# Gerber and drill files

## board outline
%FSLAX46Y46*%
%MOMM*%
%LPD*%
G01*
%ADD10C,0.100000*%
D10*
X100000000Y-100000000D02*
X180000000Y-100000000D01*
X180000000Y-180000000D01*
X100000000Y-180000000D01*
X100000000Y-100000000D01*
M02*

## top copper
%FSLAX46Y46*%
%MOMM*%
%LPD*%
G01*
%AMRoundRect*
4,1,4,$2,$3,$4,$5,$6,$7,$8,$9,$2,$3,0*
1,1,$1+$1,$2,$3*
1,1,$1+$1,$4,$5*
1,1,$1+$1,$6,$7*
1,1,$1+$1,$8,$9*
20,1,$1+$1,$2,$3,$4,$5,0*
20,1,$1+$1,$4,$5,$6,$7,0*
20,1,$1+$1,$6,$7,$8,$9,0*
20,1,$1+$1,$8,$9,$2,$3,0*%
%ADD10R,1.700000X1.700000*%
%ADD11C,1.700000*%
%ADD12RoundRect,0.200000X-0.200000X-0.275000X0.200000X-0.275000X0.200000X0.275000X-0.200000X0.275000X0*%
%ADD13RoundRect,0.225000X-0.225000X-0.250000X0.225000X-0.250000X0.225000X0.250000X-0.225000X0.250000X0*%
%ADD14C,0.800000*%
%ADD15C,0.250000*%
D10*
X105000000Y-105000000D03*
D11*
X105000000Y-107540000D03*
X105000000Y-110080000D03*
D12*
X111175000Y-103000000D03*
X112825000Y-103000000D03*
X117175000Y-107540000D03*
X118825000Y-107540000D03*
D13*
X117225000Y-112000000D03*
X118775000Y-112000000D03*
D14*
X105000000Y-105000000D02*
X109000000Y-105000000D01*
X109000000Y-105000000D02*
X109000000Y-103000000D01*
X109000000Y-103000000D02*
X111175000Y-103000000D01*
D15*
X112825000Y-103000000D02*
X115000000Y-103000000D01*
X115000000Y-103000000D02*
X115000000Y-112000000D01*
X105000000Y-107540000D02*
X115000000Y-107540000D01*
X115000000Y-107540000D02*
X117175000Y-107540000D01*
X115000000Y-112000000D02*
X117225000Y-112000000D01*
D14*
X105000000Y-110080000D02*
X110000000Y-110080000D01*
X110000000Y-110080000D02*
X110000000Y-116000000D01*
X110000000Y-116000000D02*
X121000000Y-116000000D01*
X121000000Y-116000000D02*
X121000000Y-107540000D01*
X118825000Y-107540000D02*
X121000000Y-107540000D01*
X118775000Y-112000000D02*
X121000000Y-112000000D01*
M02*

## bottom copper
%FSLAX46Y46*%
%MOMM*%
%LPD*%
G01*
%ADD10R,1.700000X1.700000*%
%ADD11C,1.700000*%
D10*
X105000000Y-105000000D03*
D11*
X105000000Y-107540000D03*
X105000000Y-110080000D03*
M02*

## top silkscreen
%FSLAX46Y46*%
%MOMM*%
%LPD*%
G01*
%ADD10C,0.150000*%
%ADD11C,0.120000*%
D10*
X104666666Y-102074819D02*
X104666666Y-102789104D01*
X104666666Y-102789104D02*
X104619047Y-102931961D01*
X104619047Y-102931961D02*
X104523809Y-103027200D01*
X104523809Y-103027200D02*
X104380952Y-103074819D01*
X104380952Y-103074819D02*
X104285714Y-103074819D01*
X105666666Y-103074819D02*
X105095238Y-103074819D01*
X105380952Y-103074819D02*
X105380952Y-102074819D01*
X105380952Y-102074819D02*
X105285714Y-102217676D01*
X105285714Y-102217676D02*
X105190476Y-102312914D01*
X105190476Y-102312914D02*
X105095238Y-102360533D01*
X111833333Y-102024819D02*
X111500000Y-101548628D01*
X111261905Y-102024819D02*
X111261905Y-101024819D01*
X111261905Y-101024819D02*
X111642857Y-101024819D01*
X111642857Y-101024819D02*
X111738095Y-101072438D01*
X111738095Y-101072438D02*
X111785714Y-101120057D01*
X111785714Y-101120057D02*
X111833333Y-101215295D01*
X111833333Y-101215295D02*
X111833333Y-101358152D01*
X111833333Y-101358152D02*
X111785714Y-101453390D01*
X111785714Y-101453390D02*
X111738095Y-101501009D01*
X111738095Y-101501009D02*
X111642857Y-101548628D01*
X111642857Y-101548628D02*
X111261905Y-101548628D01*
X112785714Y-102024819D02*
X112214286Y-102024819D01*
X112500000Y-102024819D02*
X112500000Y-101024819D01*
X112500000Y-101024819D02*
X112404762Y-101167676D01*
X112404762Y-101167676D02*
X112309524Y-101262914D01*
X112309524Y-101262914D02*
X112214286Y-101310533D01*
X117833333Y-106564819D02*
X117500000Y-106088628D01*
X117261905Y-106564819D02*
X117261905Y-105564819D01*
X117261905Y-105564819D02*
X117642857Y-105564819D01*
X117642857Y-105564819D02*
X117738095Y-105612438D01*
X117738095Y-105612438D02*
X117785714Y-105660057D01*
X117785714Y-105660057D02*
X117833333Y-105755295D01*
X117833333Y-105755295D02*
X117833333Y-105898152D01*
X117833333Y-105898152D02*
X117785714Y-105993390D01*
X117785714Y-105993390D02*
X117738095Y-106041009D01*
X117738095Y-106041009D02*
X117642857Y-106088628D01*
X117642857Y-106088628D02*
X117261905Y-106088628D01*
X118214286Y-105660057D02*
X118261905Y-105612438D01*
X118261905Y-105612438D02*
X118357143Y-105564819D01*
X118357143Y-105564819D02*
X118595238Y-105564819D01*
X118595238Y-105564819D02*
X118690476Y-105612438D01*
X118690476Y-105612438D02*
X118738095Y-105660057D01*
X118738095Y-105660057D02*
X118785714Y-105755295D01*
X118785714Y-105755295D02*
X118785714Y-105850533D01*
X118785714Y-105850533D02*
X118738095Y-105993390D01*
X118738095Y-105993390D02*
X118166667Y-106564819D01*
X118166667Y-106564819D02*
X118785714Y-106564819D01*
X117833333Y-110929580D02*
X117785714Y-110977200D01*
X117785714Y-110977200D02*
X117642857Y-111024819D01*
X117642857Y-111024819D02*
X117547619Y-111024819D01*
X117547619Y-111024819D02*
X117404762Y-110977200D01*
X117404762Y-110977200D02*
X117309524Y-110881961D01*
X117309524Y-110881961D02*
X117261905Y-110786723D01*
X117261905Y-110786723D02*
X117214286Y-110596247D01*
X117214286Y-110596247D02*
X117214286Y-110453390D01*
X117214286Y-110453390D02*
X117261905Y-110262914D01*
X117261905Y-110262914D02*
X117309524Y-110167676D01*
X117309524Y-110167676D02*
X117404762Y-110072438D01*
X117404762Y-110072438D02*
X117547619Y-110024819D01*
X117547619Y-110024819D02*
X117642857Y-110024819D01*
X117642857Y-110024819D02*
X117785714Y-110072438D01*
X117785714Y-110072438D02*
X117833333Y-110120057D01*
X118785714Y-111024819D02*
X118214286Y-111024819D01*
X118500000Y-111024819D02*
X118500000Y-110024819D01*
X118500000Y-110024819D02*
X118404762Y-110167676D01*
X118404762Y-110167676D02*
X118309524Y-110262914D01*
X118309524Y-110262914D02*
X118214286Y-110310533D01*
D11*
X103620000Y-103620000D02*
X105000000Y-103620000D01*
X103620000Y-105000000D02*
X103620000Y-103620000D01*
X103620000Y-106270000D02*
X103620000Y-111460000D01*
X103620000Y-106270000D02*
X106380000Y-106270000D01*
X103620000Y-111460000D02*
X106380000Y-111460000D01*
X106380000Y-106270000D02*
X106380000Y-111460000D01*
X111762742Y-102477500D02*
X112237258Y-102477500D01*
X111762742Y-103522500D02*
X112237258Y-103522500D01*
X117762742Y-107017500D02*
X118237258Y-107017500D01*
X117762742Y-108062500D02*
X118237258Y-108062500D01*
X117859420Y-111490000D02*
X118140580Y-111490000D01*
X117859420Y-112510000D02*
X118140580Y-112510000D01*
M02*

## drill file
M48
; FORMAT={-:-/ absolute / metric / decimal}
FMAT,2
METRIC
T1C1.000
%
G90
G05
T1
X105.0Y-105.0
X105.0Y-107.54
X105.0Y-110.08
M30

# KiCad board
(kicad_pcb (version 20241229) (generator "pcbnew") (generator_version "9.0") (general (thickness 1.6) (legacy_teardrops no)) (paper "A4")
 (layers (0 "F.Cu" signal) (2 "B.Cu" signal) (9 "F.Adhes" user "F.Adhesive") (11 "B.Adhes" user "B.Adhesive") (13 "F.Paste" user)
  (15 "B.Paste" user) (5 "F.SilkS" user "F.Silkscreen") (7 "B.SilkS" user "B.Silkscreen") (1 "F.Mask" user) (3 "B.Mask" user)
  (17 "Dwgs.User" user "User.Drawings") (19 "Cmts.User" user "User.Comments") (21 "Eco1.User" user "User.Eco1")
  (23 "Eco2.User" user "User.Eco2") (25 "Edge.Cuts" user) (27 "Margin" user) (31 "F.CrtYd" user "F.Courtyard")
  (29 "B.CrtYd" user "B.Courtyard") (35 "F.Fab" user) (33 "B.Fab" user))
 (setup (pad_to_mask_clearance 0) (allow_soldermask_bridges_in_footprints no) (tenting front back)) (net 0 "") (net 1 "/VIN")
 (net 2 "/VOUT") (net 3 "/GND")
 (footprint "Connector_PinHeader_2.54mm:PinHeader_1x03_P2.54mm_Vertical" (layer "F.Cu") (at 105 105)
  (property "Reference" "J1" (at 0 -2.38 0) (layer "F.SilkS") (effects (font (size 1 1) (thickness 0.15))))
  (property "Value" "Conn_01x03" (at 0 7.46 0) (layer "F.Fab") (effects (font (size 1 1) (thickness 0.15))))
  (fp_line (start -1.38 -1.38) (end 0 -1.38) (stroke (width 0.12) (type solid)) (layer "F.SilkS"))
  (fp_line (start -1.38 0) (end -1.38 -1.38) (stroke (width 0.12) (type solid)) (layer "F.SilkS"))
  (fp_line (start -1.38 1.27) (end -1.38 6.46) (stroke (width 0.12) (type solid)) (layer "F.SilkS"))
  (fp_line (start -1.38 1.27) (end 1.38 1.27) (stroke (width 0.12) (type solid)) (layer "F.SilkS"))
  (fp_line (start -1.38 6.46) (end 1.38 6.46) (stroke (width 0.12) (type solid)) (layer "F.SilkS"))
  (fp_line (start 1.38 1.27) (end 1.38 6.46) (stroke (width 0.12) (type solid)) (layer "F.SilkS"))
  (pad "1" thru_hole rect (at 0 0) (size 1.7 1.7) (drill 1) (layers "*.Cu" "*.Mask") (remove_unused_layers no) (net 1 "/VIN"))
  (pad "2" thru_hole circle (at 0 2.54) (size 1.7 1.7) (drill 1) (layers "*.Cu" "*.Mask") (remove_unused_layers no) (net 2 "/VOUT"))
  (pad "3" thru_hole circle (at 0 5.08) (size 1.7 1.7) (drill 1) (layers "*.Cu" "*.Mask") (remove_unused_layers no) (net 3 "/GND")))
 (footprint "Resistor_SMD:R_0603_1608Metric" (layer "F.Cu") (at 112 103)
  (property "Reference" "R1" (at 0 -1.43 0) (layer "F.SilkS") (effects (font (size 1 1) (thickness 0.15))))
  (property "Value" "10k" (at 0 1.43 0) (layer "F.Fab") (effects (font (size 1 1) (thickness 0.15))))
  (fp_line (start -0.237258 -0.5225) (end 0.237258 -0.5225) (stroke (width 0.12) (type solid)) (layer "F.SilkS"))
  (fp_line (start -0.237258 0.5225) (end 0.237258 0.5225) (stroke (width 0.12) (type solid)) (layer "F.SilkS"))
  (pad "1" smd roundrect (at -0.825 0) (size 0.8 0.95) (layers "F.Cu" "F.Mask" "F.Paste") (roundrect_rratio 0.25) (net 1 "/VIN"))
  (pad "2" smd roundrect (at 0.825 0) (size 0.8 0.95) (layers "F.Cu" "F.Mask" "F.Paste") (roundrect_rratio 0.25) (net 2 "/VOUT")))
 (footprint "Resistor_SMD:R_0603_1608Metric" (layer "F.Cu") (at 118 107.54)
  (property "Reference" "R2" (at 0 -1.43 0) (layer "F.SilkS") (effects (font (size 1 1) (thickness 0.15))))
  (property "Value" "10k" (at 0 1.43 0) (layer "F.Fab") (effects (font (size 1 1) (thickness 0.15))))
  (fp_line (start -0.237258 -0.5225) (end 0.237258 -0.5225) (stroke (width 0.12) (type solid)) (layer "F.SilkS"))
  (fp_line (start -0.237258 0.5225) (end 0.237258 0.5225) (stroke (width 0.12) (type solid)) (layer "F.SilkS"))
  (pad "1" smd roundrect (at -0.825 0) (size 0.8 0.95) (layers "F.Cu" "F.Mask" "F.Paste") (roundrect_rratio 0.25) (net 2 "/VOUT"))
  (pad "2" smd roundrect (at 0.825 0) (size 0.8 0.95) (layers "F.Cu" "F.Mask" "F.Paste") (roundrect_rratio 0.25) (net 3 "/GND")))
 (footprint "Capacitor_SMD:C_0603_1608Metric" (layer "F.Cu") (at 118 112)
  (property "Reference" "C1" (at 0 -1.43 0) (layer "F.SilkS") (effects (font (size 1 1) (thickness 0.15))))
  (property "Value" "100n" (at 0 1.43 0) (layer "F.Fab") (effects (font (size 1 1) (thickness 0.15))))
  (fp_line (start -0.14058 -0.51) (end 0.14058 -0.51) (stroke (width 0.12) (type solid)) (layer "F.SilkS"))
  (fp_line (start -0.14058 0.51) (end 0.14058 0.51) (stroke (width 0.12) (type solid)) (layer "F.SilkS"))
  (pad "1" smd roundrect (at -0.775 0) (size 0.9 0.95) (layers "F.Cu" "F.Mask" "F.Paste") (roundrect_rratio 0.25) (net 2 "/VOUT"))
  (pad "2" smd roundrect (at 0.775 0) (size 0.9 0.95) (layers "F.Cu" "F.Mask" "F.Paste") (roundrect_rratio 0.25) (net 3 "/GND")))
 (gr_rect (start 100 100) (end 180 180) (stroke (width 0.1) (type default)) (fill no) (layer "Edge.Cuts"))
 (segment (start 105 105) (end 109 105) (width 0.8) (layer "F.Cu") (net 1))
 (segment (start 109 105) (end 109 103) (width 0.8) (layer "F.Cu") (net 1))
 (segment (start 109 103) (end 111.175 103) (width 0.8) (layer "F.Cu") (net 1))
 (segment (start 112.825 103) (end 115 103) (width 0.25) (layer "F.Cu") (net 2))
 (segment (start 115 103) (end 115 112) (width 0.25) (layer "F.Cu") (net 2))
 (segment (start 105 107.54) (end 115 107.54) (width 0.25) (layer "F.Cu") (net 2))
 (segment (start 115 107.54) (end 117.175 107.54) (width 0.25) (layer "F.Cu") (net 2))
 (segment (start 115 112) (end 117.225 112) (width 0.25) (layer "F.Cu") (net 2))
 (segment (start 105 110.08) (end 110 110.08) (width 0.8) (layer "F.Cu") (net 3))
 (segment (start 110 110.08) (end 110 116) (width 0.8) (layer "F.Cu") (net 3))
 (segment (start 110 116) (end 121 116) (width 0.8) (layer "F.Cu") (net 3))
 (segment (start 121 116) (end 121 107.54) (width 0.8) (layer "F.Cu") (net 3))
 (segment (start 118.825 107.54) (end 121 107.54) (width 0.8) (layer "F.Cu") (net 3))
 (segment (start 118.775 112) (end 121 112) (width 0.8) (layer "F.Cu") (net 3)))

